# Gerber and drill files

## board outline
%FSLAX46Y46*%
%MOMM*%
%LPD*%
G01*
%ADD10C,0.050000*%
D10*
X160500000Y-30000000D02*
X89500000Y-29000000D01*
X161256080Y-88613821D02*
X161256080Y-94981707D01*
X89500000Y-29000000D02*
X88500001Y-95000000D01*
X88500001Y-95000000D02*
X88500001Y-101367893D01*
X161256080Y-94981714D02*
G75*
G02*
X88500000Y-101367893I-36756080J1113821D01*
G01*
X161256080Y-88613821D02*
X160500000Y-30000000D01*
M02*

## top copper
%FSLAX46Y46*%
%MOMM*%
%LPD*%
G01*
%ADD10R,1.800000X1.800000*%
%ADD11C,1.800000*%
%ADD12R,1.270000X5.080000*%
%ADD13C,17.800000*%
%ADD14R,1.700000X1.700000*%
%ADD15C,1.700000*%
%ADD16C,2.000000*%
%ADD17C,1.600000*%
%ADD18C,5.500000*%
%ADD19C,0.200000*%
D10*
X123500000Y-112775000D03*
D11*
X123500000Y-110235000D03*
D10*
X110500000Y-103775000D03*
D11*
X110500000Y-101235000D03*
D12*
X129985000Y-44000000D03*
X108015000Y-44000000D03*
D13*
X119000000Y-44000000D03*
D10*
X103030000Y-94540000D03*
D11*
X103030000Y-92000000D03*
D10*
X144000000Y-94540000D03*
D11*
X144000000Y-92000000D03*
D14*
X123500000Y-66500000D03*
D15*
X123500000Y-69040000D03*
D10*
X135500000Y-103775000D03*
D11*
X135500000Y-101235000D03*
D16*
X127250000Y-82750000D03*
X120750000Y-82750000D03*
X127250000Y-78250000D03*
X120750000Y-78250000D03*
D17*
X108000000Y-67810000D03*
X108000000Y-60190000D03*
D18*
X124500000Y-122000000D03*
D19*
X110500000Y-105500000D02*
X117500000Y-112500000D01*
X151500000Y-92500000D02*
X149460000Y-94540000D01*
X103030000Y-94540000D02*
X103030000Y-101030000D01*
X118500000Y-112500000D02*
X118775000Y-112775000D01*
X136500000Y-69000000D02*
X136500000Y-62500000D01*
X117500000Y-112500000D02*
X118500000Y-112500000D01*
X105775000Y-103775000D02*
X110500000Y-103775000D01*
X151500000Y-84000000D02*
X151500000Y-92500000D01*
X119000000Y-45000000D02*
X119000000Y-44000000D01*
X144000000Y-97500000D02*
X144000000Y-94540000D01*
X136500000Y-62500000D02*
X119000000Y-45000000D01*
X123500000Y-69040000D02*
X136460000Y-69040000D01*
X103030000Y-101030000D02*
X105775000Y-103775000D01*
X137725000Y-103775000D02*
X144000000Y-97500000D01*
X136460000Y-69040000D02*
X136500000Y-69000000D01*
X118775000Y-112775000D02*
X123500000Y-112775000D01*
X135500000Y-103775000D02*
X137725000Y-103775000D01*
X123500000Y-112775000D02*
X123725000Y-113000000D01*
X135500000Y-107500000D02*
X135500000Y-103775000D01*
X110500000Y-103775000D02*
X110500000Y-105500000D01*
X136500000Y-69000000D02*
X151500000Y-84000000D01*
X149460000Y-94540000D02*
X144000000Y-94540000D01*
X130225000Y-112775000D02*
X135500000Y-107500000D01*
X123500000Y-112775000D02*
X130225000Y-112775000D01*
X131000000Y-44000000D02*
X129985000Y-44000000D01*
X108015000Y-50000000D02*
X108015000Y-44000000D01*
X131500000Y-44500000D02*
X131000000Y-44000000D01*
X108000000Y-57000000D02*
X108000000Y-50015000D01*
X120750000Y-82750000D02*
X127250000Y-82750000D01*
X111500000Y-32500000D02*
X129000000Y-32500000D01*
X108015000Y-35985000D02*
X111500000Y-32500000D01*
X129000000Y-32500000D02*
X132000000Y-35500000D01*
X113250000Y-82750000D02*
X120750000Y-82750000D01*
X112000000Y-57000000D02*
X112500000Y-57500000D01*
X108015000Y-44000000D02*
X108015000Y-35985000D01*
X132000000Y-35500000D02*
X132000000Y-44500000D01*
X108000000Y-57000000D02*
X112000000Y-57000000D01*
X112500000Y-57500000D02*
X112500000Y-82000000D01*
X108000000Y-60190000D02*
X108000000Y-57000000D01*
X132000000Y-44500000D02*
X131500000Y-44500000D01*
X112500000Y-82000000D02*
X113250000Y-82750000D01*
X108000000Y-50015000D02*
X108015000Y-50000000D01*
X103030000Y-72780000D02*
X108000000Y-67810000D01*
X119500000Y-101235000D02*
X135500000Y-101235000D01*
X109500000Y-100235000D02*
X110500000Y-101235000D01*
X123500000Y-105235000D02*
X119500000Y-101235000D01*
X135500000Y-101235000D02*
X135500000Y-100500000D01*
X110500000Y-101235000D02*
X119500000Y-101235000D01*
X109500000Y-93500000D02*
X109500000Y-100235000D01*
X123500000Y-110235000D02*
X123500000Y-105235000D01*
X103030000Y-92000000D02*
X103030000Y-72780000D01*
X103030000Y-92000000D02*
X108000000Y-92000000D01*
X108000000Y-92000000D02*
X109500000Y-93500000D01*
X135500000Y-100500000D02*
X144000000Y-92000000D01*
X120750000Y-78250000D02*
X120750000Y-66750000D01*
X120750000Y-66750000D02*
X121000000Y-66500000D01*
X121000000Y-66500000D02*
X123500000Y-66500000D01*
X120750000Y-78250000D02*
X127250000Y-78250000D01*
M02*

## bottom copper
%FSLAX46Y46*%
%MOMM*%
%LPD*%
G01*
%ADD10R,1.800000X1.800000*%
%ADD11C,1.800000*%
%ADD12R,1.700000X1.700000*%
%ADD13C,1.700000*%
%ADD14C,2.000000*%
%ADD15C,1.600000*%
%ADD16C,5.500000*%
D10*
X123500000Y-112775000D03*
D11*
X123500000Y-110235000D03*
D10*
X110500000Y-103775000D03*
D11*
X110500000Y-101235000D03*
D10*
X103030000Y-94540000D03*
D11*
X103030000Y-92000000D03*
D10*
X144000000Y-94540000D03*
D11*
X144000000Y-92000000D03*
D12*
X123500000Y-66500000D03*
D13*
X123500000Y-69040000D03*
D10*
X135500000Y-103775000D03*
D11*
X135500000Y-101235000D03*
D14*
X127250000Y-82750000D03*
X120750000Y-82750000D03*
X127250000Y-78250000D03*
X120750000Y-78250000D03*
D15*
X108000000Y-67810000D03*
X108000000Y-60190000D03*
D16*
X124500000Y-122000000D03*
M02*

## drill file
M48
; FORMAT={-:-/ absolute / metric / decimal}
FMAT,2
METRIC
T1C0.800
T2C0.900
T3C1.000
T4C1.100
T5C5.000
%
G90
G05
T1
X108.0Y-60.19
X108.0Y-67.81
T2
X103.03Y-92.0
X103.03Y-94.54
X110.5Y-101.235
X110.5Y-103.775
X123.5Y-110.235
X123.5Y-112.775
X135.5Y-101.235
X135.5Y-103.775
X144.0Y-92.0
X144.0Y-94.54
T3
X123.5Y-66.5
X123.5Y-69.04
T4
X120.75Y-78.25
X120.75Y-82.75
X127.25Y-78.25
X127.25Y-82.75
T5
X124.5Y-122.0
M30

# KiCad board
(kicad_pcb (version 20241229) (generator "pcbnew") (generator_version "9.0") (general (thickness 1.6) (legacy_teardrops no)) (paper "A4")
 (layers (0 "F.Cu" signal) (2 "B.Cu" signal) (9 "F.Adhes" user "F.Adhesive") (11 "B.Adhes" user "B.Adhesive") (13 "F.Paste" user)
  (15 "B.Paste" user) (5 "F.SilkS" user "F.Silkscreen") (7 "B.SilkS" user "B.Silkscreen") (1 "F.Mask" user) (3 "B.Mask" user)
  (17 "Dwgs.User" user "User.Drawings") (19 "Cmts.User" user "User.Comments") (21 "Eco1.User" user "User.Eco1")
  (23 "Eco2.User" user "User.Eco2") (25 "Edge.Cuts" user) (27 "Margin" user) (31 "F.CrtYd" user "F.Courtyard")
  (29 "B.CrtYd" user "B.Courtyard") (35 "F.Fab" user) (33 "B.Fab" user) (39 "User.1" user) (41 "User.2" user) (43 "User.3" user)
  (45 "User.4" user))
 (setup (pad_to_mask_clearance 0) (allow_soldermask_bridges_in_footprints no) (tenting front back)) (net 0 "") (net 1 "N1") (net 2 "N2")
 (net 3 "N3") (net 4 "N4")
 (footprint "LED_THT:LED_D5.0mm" (layer "F.Cu") (at 123.5 112.775 90)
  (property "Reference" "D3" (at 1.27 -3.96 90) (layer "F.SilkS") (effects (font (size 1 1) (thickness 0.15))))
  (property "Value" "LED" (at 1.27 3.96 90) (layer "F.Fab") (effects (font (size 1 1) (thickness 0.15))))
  (pad "1" thru_hole rect (at 0 0 90) (size 1.8 1.8) (drill 0.9) (layers "*.Cu" "*.Mask") (remove_unused_layers no) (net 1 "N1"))
  (pad "2" thru_hole circle (at 2.54 0 90) (size 1.8 1.8) (drill 0.9) (layers "*.Cu" "*.Mask") (remove_unused_layers no) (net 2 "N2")))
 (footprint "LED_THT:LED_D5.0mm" (layer "F.Cu") (at 110.5 103.775 90)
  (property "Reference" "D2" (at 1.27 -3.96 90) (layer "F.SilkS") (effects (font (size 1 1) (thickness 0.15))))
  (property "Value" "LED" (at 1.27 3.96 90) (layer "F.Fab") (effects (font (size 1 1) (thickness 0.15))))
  (pad "1" thru_hole rect (at 0 0 90) (size 1.8 1.8) (drill 0.9) (layers "*.Cu" "*.Mask") (remove_unused_layers no) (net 1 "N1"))
  (pad "2" thru_hole circle (at 2.54 0 90) (size 1.8 1.8) (drill 0.9) (layers "*.Cu" "*.Mask") (remove_unused_layers no) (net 2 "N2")))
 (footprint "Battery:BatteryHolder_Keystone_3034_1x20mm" (layer "F.Cu") (at 119 44 180)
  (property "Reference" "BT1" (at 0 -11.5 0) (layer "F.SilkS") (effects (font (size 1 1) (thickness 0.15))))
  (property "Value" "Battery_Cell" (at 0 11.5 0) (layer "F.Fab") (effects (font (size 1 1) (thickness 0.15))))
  (pad "1" smd rect (at -10.985 0 180) (size 1.27 5.08) (layers "F.Cu" "F.Mask" "F.Paste") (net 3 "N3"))
  (pad "1" smd rect (at 10.985 0 180) (size 1.27 5.08) (layers "F.Cu" "F.Mask" "F.Paste") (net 3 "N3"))
  (pad "2" smd circle (at 0 0 180) (size 17.8 17.8) (layers "F.Cu" "F.Mask") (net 1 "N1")))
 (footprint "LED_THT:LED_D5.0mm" (layer "F.Cu") (at 103.03 94.54 90)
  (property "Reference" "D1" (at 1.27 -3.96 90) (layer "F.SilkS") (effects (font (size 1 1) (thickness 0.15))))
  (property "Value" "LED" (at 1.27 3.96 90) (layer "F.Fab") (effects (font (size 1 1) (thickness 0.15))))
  (pad "1" thru_hole rect (at 0 0 90) (size 1.8 1.8) (drill 0.9) (layers "*.Cu" "*.Mask") (remove_unused_layers no) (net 1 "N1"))
  (pad "2" thru_hole circle (at 2.54 0 90) (size 1.8 1.8) (drill 0.9) (layers "*.Cu" "*.Mask") (remove_unused_layers no) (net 2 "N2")))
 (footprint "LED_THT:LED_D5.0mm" (layer "F.Cu") (at 144 94.54 90)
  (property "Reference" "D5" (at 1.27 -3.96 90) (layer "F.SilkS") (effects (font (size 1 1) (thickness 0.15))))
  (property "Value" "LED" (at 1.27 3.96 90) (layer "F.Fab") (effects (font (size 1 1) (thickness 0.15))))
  (pad "1" thru_hole rect (at 0 0 90) (size 1.8 1.8) (drill 0.9) (layers "*.Cu" "*.Mask") (remove_unused_layers no) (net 1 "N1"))
  (pad "2" thru_hole circle (at 2.54 0 90) (size 1.8 1.8) (drill 0.9) (layers "*.Cu" "*.Mask") (remove_unused_layers no) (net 2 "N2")))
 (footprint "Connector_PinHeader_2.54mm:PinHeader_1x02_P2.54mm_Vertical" (layer "F.Cu") (at 123.5 66.5)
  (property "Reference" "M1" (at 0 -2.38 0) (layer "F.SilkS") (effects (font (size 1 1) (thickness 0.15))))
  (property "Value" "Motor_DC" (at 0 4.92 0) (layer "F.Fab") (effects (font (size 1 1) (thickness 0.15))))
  (pad "1" thru_hole rect (at 0 0) (size 1.7 1.7) (drill 1) (layers "*.Cu" "*.Mask") (remove_unused_layers no) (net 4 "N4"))
  (pad "2" thru_hole circle (at 0 2.54) (size 1.7 1.7) (drill 1) (layers "*.Cu" "*.Mask") (remove_unused_layers no) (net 1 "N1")))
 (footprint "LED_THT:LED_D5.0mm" (layer "F.Cu") (at 135.5 103.775 90)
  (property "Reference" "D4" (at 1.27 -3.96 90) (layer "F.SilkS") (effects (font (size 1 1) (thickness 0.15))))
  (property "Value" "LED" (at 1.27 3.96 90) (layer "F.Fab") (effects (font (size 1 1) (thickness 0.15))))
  (pad "1" thru_hole rect (at 0 0 90) (size 1.8 1.8) (drill 0.9) (layers "*.Cu" "*.Mask") (remove_unused_layers no) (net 1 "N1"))
  (pad "2" thru_hole circle (at 2.54 0 90) (size 1.8 1.8) (drill 0.9) (layers "*.Cu" "*.Mask") (remove_unused_layers no) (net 2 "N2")))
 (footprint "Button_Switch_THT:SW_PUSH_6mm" (layer "F.Cu") (at 127.25 82.75 180)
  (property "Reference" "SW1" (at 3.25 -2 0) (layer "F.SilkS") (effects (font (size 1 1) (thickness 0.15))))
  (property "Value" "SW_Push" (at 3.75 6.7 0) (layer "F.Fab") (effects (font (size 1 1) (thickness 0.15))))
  (pad "1" thru_hole circle (at 0 0 270) (size 2 2) (drill 1.1) (layers "*.Cu" "*.Mask") (remove_unused_layers no) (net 3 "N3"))
  (pad "1" thru_hole circle (at 6.5 0 270) (size 2 2) (drill 1.1) (layers "*.Cu" "*.Mask") (remove_unused_layers no) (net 3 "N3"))
  (pad "2" thru_hole circle (at 0 4.5 270) (size 2 2) (drill 1.1) (layers "*.Cu" "*.Mask") (remove_unused_layers no) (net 4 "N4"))
  (pad "2" thru_hole circle (at 6.5 4.5 270) (size 2 2) (drill 1.1) (layers "*.Cu" "*.Mask") (remove_unused_layers no) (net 4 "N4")))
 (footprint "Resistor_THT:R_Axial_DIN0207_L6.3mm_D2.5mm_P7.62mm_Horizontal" (layer "F.Cu") (at 108 67.81 90)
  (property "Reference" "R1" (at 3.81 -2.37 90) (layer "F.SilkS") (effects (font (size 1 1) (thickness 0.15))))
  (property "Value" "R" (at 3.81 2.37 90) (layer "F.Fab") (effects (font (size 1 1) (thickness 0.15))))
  (pad "1" thru_hole circle (at 0 0 90) (size 1.6 1.6) (drill 0.8) (layers "*.Cu" "*.Mask") (remove_unused_layers no) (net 2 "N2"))
  (pad "2" thru_hole circle (at 7.62 0 90) (size 1.6 1.6) (drill 0.8) (layers "*.Cu" "*.Mask") (remove_unused_layers no) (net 3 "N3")))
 (gr_line (start 160.5 30) (end 89.5 29) (stroke (width 0.05) (type default)) (layer "Edge.Cuts"))
 (gr_line (start 161.25608 88.613821) (end 161.25608 94.981707) (stroke (width 0.05) (type default)) (layer "Edge.Cuts"))
 (gr_line (start 89.5 29) (end 88.500001 95) (stroke (width 0.05) (type default)) (layer "Edge.Cuts"))
 (gr_line (start 88.500001 95) (end 88.500001 101.367893) (stroke (width 0.05) (type default)) (layer "Edge.Cuts"))
 (gr_arc (start 161.25608 94.981714) (mid 127.71539 130.5) (end 88.5 101.367893) (stroke (width 0.05) (type default)) (layer "Edge.Cuts"))
 (gr_line (start 161.25608 88.613821) (end 160.5 30) (stroke (width 0.05) (type default)) (layer "Edge.Cuts"))
 (via (at 124.5 122) (size 5.5) (drill 5) (layers "F.Cu" "B.Cu") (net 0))
 (segment (start 110.5 105.5) (end 117.5 112.5) (width 0.2) (layer "F.Cu") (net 1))
 (segment (start 151.5 92.5) (end 149.46 94.54) (width 0.2) (layer "F.Cu") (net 1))
 (segment (start 103.03 94.54) (end 103.03 101.03) (width 0.2) (layer "F.Cu") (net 1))
 (segment (start 118.5 112.5) (end 118.775 112.775) (width 0.2) (layer "F.Cu") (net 1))
 (segment (start 136.5 69) (end 136.5 62.5) (width 0.2) (layer "F.Cu") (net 1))
 (segment (start 117.5 112.5) (end 118.5 112.5) (width 0.2) (layer "F.Cu") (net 1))
 (segment (start 105.775 103.775) (end 110.5 103.775) (width 0.2) (layer "F.Cu") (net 1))
 (segment (start 151.5 84) (end 151.5 92.5) (width 0.2) (layer "F.Cu") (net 1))
 (segment (start 119 45) (end 119 44) (width 0.2) (layer "F.Cu") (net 1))
 (segment (start 144 97.5) (end 144 94.54) (width 0.2) (layer "F.Cu") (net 1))
 (segment (start 136.5 62.5) (end 119 45) (width 0.2) (layer "F.Cu") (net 1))
 (segment (start 123.5 69.04) (end 136.46 69.04) (width 0.2) (layer "F.Cu") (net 1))
 (segment (start 103.03 101.03) (end 105.775 103.775) (width 0.2) (layer "F.Cu") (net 1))
 (segment (start 137.725 103.775) (end 144 97.5) (width 0.2) (layer "F.Cu") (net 1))
 (segment (start 136.46 69.04) (end 136.5 69) (width 0.2) (layer "F.Cu") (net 1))
 (segment (start 118.775 112.775) (end 123.5 112.775) (width 0.2) (layer "F.Cu") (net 1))
 (segment (start 135.5 103.775) (end 137.725 103.775) (width 0.2) (layer "F.Cu") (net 1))
 (segment (start 123.5 112.775) (end 123.725 113) (width 0.2) (layer "F.Cu") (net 1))
 (segment (start 135.5 107.5) (end 135.5 103.775) (width 0.2) (layer "F.Cu") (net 1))
 (segment (start 110.5 103.775) (end 110.5 105.5) (width 0.2) (layer "F.Cu") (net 1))
 (segment (start 136.5 69) (end 151.5 84) (width 0.2) (layer "F.Cu") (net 1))
 (segment (start 149.46 94.54) (end 144 94.54) (width 0.2) (layer "F.Cu") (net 1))
 (segment (start 130.225 112.775) (end 135.5 107.5) (width 0.2) (layer "F.Cu") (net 1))
 (segment (start 123.5 112.775) (end 130.225 112.775) (width 0.2) (layer "F.Cu") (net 1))
 (segment (start 131 44) (end 129.985 44) (width 0.2) (layer "F.Cu") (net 3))
 (segment (start 108.015 50) (end 108.015 44) (width 0.2) (layer "F.Cu") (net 3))
 (segment (start 131.5 44.5) (end 131 44) (width 0.2) (layer "F.Cu") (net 3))
 (segment (start 108 57) (end 108 50.015) (width 0.2) (layer "F.Cu") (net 3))
 (segment (start 120.75 82.75) (end 127.25 82.75) (width 0.2) (layer "F.Cu") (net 3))
 (segment (start 111.5 32.5) (end 129 32.5) (width 0.2) (layer "F.Cu") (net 3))
 (segment (start 108.015 35.985) (end 111.5 32.5) (width 0.2) (layer "F.Cu") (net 3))
 (segment (start 129 32.5) (end 132 35.5) (width 0.2) (layer "F.Cu") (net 3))
 (segment (start 113.25 82.75) (end 120.75 82.75) (width 0.2) (layer "F.Cu") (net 3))
 (segment (start 112 57) (end 112.5 57.5) (width 0.2) (layer "F.Cu") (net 3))
 (segment (start 108.015 44) (end 108.015 35.985) (width 0.2) (layer "F.Cu") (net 3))
 (segment (start 132 35.5) (end 132 44.5) (width 0.2) (layer "F.Cu") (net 3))
 (segment (start 108 57) (end 112 57) (width 0.2) (layer "F.Cu") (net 3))
 (segment (start 112.5 57.5) (end 112.5 82) (width 0.2) (layer "F.Cu") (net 3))
 (segment (start 108 60.19) (end 108 57) (width 0.2) (layer "F.Cu") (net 3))
 (segment (start 132 44.5) (end 131.5 44.5) (width 0.2) (layer "F.Cu") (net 3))
 (segment (start 112.5 82) (end 113.25 82.75) (width 0.2) (layer "F.Cu") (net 3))
 (segment (start 108 50.015) (end 108.015 50) (width 0.2) (layer "F.Cu") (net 3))
 (segment (start 103.03 72.78) (end 108 67.81) (width 0.2) (layer "F.Cu") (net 2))
 (segment (start 119.5 101.235) (end 135.5 101.235) (width 0.2) (layer "F.Cu") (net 2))
 (segment (start 109.5 100.235) (end 110.5 101.235) (width 0.2) (layer "F.Cu") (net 2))
 (segment (start 123.5 105.235) (end 119.5 101.235) (width 0.2) (layer "F.Cu") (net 2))
 (segment (start 135.5 101.235) (end 135.5 100.5) (width 0.2) (layer "F.Cu") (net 2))
 (segment (start 110.5 101.235) (end 119.5 101.235) (width 0.2) (layer "F.Cu") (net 2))
 (segment (start 109.5 93.5) (end 109.5 100.235) (width 0.2) (layer "F.Cu") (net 2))
 (segment (start 123.5 110.235) (end 123.5 105.235) (width 0.2) (layer "F.Cu") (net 2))
 (segment (start 103.03 92) (end 103.03 72.78) (width 0.2) (layer "F.Cu") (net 2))
 (segment (start 103.03 92) (end 108 92) (width 0.2) (layer "F.Cu") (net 2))
 (segment (start 108 92) (end 109.5 93.5) (width 0.2) (layer "F.Cu") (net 2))
 (segment (start 135.5 100.5) (end 144 92) (width 0.2) (layer "F.Cu") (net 2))
 (segment (start 120.75 78.25) (end 120.75 66.75) (width 0.2) (layer "F.Cu") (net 4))
 (segment (start 120.75 66.75) (end 121 66.5) (width 0.2) (layer "F.Cu") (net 4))
 (segment (start 121 66.5) (end 123.5 66.5) (width 0.2) (layer "F.Cu") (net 4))
 (segment (start 120.75 78.25) (end 127.25 78.25) (width 0.2) (layer "F.Cu") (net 4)))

